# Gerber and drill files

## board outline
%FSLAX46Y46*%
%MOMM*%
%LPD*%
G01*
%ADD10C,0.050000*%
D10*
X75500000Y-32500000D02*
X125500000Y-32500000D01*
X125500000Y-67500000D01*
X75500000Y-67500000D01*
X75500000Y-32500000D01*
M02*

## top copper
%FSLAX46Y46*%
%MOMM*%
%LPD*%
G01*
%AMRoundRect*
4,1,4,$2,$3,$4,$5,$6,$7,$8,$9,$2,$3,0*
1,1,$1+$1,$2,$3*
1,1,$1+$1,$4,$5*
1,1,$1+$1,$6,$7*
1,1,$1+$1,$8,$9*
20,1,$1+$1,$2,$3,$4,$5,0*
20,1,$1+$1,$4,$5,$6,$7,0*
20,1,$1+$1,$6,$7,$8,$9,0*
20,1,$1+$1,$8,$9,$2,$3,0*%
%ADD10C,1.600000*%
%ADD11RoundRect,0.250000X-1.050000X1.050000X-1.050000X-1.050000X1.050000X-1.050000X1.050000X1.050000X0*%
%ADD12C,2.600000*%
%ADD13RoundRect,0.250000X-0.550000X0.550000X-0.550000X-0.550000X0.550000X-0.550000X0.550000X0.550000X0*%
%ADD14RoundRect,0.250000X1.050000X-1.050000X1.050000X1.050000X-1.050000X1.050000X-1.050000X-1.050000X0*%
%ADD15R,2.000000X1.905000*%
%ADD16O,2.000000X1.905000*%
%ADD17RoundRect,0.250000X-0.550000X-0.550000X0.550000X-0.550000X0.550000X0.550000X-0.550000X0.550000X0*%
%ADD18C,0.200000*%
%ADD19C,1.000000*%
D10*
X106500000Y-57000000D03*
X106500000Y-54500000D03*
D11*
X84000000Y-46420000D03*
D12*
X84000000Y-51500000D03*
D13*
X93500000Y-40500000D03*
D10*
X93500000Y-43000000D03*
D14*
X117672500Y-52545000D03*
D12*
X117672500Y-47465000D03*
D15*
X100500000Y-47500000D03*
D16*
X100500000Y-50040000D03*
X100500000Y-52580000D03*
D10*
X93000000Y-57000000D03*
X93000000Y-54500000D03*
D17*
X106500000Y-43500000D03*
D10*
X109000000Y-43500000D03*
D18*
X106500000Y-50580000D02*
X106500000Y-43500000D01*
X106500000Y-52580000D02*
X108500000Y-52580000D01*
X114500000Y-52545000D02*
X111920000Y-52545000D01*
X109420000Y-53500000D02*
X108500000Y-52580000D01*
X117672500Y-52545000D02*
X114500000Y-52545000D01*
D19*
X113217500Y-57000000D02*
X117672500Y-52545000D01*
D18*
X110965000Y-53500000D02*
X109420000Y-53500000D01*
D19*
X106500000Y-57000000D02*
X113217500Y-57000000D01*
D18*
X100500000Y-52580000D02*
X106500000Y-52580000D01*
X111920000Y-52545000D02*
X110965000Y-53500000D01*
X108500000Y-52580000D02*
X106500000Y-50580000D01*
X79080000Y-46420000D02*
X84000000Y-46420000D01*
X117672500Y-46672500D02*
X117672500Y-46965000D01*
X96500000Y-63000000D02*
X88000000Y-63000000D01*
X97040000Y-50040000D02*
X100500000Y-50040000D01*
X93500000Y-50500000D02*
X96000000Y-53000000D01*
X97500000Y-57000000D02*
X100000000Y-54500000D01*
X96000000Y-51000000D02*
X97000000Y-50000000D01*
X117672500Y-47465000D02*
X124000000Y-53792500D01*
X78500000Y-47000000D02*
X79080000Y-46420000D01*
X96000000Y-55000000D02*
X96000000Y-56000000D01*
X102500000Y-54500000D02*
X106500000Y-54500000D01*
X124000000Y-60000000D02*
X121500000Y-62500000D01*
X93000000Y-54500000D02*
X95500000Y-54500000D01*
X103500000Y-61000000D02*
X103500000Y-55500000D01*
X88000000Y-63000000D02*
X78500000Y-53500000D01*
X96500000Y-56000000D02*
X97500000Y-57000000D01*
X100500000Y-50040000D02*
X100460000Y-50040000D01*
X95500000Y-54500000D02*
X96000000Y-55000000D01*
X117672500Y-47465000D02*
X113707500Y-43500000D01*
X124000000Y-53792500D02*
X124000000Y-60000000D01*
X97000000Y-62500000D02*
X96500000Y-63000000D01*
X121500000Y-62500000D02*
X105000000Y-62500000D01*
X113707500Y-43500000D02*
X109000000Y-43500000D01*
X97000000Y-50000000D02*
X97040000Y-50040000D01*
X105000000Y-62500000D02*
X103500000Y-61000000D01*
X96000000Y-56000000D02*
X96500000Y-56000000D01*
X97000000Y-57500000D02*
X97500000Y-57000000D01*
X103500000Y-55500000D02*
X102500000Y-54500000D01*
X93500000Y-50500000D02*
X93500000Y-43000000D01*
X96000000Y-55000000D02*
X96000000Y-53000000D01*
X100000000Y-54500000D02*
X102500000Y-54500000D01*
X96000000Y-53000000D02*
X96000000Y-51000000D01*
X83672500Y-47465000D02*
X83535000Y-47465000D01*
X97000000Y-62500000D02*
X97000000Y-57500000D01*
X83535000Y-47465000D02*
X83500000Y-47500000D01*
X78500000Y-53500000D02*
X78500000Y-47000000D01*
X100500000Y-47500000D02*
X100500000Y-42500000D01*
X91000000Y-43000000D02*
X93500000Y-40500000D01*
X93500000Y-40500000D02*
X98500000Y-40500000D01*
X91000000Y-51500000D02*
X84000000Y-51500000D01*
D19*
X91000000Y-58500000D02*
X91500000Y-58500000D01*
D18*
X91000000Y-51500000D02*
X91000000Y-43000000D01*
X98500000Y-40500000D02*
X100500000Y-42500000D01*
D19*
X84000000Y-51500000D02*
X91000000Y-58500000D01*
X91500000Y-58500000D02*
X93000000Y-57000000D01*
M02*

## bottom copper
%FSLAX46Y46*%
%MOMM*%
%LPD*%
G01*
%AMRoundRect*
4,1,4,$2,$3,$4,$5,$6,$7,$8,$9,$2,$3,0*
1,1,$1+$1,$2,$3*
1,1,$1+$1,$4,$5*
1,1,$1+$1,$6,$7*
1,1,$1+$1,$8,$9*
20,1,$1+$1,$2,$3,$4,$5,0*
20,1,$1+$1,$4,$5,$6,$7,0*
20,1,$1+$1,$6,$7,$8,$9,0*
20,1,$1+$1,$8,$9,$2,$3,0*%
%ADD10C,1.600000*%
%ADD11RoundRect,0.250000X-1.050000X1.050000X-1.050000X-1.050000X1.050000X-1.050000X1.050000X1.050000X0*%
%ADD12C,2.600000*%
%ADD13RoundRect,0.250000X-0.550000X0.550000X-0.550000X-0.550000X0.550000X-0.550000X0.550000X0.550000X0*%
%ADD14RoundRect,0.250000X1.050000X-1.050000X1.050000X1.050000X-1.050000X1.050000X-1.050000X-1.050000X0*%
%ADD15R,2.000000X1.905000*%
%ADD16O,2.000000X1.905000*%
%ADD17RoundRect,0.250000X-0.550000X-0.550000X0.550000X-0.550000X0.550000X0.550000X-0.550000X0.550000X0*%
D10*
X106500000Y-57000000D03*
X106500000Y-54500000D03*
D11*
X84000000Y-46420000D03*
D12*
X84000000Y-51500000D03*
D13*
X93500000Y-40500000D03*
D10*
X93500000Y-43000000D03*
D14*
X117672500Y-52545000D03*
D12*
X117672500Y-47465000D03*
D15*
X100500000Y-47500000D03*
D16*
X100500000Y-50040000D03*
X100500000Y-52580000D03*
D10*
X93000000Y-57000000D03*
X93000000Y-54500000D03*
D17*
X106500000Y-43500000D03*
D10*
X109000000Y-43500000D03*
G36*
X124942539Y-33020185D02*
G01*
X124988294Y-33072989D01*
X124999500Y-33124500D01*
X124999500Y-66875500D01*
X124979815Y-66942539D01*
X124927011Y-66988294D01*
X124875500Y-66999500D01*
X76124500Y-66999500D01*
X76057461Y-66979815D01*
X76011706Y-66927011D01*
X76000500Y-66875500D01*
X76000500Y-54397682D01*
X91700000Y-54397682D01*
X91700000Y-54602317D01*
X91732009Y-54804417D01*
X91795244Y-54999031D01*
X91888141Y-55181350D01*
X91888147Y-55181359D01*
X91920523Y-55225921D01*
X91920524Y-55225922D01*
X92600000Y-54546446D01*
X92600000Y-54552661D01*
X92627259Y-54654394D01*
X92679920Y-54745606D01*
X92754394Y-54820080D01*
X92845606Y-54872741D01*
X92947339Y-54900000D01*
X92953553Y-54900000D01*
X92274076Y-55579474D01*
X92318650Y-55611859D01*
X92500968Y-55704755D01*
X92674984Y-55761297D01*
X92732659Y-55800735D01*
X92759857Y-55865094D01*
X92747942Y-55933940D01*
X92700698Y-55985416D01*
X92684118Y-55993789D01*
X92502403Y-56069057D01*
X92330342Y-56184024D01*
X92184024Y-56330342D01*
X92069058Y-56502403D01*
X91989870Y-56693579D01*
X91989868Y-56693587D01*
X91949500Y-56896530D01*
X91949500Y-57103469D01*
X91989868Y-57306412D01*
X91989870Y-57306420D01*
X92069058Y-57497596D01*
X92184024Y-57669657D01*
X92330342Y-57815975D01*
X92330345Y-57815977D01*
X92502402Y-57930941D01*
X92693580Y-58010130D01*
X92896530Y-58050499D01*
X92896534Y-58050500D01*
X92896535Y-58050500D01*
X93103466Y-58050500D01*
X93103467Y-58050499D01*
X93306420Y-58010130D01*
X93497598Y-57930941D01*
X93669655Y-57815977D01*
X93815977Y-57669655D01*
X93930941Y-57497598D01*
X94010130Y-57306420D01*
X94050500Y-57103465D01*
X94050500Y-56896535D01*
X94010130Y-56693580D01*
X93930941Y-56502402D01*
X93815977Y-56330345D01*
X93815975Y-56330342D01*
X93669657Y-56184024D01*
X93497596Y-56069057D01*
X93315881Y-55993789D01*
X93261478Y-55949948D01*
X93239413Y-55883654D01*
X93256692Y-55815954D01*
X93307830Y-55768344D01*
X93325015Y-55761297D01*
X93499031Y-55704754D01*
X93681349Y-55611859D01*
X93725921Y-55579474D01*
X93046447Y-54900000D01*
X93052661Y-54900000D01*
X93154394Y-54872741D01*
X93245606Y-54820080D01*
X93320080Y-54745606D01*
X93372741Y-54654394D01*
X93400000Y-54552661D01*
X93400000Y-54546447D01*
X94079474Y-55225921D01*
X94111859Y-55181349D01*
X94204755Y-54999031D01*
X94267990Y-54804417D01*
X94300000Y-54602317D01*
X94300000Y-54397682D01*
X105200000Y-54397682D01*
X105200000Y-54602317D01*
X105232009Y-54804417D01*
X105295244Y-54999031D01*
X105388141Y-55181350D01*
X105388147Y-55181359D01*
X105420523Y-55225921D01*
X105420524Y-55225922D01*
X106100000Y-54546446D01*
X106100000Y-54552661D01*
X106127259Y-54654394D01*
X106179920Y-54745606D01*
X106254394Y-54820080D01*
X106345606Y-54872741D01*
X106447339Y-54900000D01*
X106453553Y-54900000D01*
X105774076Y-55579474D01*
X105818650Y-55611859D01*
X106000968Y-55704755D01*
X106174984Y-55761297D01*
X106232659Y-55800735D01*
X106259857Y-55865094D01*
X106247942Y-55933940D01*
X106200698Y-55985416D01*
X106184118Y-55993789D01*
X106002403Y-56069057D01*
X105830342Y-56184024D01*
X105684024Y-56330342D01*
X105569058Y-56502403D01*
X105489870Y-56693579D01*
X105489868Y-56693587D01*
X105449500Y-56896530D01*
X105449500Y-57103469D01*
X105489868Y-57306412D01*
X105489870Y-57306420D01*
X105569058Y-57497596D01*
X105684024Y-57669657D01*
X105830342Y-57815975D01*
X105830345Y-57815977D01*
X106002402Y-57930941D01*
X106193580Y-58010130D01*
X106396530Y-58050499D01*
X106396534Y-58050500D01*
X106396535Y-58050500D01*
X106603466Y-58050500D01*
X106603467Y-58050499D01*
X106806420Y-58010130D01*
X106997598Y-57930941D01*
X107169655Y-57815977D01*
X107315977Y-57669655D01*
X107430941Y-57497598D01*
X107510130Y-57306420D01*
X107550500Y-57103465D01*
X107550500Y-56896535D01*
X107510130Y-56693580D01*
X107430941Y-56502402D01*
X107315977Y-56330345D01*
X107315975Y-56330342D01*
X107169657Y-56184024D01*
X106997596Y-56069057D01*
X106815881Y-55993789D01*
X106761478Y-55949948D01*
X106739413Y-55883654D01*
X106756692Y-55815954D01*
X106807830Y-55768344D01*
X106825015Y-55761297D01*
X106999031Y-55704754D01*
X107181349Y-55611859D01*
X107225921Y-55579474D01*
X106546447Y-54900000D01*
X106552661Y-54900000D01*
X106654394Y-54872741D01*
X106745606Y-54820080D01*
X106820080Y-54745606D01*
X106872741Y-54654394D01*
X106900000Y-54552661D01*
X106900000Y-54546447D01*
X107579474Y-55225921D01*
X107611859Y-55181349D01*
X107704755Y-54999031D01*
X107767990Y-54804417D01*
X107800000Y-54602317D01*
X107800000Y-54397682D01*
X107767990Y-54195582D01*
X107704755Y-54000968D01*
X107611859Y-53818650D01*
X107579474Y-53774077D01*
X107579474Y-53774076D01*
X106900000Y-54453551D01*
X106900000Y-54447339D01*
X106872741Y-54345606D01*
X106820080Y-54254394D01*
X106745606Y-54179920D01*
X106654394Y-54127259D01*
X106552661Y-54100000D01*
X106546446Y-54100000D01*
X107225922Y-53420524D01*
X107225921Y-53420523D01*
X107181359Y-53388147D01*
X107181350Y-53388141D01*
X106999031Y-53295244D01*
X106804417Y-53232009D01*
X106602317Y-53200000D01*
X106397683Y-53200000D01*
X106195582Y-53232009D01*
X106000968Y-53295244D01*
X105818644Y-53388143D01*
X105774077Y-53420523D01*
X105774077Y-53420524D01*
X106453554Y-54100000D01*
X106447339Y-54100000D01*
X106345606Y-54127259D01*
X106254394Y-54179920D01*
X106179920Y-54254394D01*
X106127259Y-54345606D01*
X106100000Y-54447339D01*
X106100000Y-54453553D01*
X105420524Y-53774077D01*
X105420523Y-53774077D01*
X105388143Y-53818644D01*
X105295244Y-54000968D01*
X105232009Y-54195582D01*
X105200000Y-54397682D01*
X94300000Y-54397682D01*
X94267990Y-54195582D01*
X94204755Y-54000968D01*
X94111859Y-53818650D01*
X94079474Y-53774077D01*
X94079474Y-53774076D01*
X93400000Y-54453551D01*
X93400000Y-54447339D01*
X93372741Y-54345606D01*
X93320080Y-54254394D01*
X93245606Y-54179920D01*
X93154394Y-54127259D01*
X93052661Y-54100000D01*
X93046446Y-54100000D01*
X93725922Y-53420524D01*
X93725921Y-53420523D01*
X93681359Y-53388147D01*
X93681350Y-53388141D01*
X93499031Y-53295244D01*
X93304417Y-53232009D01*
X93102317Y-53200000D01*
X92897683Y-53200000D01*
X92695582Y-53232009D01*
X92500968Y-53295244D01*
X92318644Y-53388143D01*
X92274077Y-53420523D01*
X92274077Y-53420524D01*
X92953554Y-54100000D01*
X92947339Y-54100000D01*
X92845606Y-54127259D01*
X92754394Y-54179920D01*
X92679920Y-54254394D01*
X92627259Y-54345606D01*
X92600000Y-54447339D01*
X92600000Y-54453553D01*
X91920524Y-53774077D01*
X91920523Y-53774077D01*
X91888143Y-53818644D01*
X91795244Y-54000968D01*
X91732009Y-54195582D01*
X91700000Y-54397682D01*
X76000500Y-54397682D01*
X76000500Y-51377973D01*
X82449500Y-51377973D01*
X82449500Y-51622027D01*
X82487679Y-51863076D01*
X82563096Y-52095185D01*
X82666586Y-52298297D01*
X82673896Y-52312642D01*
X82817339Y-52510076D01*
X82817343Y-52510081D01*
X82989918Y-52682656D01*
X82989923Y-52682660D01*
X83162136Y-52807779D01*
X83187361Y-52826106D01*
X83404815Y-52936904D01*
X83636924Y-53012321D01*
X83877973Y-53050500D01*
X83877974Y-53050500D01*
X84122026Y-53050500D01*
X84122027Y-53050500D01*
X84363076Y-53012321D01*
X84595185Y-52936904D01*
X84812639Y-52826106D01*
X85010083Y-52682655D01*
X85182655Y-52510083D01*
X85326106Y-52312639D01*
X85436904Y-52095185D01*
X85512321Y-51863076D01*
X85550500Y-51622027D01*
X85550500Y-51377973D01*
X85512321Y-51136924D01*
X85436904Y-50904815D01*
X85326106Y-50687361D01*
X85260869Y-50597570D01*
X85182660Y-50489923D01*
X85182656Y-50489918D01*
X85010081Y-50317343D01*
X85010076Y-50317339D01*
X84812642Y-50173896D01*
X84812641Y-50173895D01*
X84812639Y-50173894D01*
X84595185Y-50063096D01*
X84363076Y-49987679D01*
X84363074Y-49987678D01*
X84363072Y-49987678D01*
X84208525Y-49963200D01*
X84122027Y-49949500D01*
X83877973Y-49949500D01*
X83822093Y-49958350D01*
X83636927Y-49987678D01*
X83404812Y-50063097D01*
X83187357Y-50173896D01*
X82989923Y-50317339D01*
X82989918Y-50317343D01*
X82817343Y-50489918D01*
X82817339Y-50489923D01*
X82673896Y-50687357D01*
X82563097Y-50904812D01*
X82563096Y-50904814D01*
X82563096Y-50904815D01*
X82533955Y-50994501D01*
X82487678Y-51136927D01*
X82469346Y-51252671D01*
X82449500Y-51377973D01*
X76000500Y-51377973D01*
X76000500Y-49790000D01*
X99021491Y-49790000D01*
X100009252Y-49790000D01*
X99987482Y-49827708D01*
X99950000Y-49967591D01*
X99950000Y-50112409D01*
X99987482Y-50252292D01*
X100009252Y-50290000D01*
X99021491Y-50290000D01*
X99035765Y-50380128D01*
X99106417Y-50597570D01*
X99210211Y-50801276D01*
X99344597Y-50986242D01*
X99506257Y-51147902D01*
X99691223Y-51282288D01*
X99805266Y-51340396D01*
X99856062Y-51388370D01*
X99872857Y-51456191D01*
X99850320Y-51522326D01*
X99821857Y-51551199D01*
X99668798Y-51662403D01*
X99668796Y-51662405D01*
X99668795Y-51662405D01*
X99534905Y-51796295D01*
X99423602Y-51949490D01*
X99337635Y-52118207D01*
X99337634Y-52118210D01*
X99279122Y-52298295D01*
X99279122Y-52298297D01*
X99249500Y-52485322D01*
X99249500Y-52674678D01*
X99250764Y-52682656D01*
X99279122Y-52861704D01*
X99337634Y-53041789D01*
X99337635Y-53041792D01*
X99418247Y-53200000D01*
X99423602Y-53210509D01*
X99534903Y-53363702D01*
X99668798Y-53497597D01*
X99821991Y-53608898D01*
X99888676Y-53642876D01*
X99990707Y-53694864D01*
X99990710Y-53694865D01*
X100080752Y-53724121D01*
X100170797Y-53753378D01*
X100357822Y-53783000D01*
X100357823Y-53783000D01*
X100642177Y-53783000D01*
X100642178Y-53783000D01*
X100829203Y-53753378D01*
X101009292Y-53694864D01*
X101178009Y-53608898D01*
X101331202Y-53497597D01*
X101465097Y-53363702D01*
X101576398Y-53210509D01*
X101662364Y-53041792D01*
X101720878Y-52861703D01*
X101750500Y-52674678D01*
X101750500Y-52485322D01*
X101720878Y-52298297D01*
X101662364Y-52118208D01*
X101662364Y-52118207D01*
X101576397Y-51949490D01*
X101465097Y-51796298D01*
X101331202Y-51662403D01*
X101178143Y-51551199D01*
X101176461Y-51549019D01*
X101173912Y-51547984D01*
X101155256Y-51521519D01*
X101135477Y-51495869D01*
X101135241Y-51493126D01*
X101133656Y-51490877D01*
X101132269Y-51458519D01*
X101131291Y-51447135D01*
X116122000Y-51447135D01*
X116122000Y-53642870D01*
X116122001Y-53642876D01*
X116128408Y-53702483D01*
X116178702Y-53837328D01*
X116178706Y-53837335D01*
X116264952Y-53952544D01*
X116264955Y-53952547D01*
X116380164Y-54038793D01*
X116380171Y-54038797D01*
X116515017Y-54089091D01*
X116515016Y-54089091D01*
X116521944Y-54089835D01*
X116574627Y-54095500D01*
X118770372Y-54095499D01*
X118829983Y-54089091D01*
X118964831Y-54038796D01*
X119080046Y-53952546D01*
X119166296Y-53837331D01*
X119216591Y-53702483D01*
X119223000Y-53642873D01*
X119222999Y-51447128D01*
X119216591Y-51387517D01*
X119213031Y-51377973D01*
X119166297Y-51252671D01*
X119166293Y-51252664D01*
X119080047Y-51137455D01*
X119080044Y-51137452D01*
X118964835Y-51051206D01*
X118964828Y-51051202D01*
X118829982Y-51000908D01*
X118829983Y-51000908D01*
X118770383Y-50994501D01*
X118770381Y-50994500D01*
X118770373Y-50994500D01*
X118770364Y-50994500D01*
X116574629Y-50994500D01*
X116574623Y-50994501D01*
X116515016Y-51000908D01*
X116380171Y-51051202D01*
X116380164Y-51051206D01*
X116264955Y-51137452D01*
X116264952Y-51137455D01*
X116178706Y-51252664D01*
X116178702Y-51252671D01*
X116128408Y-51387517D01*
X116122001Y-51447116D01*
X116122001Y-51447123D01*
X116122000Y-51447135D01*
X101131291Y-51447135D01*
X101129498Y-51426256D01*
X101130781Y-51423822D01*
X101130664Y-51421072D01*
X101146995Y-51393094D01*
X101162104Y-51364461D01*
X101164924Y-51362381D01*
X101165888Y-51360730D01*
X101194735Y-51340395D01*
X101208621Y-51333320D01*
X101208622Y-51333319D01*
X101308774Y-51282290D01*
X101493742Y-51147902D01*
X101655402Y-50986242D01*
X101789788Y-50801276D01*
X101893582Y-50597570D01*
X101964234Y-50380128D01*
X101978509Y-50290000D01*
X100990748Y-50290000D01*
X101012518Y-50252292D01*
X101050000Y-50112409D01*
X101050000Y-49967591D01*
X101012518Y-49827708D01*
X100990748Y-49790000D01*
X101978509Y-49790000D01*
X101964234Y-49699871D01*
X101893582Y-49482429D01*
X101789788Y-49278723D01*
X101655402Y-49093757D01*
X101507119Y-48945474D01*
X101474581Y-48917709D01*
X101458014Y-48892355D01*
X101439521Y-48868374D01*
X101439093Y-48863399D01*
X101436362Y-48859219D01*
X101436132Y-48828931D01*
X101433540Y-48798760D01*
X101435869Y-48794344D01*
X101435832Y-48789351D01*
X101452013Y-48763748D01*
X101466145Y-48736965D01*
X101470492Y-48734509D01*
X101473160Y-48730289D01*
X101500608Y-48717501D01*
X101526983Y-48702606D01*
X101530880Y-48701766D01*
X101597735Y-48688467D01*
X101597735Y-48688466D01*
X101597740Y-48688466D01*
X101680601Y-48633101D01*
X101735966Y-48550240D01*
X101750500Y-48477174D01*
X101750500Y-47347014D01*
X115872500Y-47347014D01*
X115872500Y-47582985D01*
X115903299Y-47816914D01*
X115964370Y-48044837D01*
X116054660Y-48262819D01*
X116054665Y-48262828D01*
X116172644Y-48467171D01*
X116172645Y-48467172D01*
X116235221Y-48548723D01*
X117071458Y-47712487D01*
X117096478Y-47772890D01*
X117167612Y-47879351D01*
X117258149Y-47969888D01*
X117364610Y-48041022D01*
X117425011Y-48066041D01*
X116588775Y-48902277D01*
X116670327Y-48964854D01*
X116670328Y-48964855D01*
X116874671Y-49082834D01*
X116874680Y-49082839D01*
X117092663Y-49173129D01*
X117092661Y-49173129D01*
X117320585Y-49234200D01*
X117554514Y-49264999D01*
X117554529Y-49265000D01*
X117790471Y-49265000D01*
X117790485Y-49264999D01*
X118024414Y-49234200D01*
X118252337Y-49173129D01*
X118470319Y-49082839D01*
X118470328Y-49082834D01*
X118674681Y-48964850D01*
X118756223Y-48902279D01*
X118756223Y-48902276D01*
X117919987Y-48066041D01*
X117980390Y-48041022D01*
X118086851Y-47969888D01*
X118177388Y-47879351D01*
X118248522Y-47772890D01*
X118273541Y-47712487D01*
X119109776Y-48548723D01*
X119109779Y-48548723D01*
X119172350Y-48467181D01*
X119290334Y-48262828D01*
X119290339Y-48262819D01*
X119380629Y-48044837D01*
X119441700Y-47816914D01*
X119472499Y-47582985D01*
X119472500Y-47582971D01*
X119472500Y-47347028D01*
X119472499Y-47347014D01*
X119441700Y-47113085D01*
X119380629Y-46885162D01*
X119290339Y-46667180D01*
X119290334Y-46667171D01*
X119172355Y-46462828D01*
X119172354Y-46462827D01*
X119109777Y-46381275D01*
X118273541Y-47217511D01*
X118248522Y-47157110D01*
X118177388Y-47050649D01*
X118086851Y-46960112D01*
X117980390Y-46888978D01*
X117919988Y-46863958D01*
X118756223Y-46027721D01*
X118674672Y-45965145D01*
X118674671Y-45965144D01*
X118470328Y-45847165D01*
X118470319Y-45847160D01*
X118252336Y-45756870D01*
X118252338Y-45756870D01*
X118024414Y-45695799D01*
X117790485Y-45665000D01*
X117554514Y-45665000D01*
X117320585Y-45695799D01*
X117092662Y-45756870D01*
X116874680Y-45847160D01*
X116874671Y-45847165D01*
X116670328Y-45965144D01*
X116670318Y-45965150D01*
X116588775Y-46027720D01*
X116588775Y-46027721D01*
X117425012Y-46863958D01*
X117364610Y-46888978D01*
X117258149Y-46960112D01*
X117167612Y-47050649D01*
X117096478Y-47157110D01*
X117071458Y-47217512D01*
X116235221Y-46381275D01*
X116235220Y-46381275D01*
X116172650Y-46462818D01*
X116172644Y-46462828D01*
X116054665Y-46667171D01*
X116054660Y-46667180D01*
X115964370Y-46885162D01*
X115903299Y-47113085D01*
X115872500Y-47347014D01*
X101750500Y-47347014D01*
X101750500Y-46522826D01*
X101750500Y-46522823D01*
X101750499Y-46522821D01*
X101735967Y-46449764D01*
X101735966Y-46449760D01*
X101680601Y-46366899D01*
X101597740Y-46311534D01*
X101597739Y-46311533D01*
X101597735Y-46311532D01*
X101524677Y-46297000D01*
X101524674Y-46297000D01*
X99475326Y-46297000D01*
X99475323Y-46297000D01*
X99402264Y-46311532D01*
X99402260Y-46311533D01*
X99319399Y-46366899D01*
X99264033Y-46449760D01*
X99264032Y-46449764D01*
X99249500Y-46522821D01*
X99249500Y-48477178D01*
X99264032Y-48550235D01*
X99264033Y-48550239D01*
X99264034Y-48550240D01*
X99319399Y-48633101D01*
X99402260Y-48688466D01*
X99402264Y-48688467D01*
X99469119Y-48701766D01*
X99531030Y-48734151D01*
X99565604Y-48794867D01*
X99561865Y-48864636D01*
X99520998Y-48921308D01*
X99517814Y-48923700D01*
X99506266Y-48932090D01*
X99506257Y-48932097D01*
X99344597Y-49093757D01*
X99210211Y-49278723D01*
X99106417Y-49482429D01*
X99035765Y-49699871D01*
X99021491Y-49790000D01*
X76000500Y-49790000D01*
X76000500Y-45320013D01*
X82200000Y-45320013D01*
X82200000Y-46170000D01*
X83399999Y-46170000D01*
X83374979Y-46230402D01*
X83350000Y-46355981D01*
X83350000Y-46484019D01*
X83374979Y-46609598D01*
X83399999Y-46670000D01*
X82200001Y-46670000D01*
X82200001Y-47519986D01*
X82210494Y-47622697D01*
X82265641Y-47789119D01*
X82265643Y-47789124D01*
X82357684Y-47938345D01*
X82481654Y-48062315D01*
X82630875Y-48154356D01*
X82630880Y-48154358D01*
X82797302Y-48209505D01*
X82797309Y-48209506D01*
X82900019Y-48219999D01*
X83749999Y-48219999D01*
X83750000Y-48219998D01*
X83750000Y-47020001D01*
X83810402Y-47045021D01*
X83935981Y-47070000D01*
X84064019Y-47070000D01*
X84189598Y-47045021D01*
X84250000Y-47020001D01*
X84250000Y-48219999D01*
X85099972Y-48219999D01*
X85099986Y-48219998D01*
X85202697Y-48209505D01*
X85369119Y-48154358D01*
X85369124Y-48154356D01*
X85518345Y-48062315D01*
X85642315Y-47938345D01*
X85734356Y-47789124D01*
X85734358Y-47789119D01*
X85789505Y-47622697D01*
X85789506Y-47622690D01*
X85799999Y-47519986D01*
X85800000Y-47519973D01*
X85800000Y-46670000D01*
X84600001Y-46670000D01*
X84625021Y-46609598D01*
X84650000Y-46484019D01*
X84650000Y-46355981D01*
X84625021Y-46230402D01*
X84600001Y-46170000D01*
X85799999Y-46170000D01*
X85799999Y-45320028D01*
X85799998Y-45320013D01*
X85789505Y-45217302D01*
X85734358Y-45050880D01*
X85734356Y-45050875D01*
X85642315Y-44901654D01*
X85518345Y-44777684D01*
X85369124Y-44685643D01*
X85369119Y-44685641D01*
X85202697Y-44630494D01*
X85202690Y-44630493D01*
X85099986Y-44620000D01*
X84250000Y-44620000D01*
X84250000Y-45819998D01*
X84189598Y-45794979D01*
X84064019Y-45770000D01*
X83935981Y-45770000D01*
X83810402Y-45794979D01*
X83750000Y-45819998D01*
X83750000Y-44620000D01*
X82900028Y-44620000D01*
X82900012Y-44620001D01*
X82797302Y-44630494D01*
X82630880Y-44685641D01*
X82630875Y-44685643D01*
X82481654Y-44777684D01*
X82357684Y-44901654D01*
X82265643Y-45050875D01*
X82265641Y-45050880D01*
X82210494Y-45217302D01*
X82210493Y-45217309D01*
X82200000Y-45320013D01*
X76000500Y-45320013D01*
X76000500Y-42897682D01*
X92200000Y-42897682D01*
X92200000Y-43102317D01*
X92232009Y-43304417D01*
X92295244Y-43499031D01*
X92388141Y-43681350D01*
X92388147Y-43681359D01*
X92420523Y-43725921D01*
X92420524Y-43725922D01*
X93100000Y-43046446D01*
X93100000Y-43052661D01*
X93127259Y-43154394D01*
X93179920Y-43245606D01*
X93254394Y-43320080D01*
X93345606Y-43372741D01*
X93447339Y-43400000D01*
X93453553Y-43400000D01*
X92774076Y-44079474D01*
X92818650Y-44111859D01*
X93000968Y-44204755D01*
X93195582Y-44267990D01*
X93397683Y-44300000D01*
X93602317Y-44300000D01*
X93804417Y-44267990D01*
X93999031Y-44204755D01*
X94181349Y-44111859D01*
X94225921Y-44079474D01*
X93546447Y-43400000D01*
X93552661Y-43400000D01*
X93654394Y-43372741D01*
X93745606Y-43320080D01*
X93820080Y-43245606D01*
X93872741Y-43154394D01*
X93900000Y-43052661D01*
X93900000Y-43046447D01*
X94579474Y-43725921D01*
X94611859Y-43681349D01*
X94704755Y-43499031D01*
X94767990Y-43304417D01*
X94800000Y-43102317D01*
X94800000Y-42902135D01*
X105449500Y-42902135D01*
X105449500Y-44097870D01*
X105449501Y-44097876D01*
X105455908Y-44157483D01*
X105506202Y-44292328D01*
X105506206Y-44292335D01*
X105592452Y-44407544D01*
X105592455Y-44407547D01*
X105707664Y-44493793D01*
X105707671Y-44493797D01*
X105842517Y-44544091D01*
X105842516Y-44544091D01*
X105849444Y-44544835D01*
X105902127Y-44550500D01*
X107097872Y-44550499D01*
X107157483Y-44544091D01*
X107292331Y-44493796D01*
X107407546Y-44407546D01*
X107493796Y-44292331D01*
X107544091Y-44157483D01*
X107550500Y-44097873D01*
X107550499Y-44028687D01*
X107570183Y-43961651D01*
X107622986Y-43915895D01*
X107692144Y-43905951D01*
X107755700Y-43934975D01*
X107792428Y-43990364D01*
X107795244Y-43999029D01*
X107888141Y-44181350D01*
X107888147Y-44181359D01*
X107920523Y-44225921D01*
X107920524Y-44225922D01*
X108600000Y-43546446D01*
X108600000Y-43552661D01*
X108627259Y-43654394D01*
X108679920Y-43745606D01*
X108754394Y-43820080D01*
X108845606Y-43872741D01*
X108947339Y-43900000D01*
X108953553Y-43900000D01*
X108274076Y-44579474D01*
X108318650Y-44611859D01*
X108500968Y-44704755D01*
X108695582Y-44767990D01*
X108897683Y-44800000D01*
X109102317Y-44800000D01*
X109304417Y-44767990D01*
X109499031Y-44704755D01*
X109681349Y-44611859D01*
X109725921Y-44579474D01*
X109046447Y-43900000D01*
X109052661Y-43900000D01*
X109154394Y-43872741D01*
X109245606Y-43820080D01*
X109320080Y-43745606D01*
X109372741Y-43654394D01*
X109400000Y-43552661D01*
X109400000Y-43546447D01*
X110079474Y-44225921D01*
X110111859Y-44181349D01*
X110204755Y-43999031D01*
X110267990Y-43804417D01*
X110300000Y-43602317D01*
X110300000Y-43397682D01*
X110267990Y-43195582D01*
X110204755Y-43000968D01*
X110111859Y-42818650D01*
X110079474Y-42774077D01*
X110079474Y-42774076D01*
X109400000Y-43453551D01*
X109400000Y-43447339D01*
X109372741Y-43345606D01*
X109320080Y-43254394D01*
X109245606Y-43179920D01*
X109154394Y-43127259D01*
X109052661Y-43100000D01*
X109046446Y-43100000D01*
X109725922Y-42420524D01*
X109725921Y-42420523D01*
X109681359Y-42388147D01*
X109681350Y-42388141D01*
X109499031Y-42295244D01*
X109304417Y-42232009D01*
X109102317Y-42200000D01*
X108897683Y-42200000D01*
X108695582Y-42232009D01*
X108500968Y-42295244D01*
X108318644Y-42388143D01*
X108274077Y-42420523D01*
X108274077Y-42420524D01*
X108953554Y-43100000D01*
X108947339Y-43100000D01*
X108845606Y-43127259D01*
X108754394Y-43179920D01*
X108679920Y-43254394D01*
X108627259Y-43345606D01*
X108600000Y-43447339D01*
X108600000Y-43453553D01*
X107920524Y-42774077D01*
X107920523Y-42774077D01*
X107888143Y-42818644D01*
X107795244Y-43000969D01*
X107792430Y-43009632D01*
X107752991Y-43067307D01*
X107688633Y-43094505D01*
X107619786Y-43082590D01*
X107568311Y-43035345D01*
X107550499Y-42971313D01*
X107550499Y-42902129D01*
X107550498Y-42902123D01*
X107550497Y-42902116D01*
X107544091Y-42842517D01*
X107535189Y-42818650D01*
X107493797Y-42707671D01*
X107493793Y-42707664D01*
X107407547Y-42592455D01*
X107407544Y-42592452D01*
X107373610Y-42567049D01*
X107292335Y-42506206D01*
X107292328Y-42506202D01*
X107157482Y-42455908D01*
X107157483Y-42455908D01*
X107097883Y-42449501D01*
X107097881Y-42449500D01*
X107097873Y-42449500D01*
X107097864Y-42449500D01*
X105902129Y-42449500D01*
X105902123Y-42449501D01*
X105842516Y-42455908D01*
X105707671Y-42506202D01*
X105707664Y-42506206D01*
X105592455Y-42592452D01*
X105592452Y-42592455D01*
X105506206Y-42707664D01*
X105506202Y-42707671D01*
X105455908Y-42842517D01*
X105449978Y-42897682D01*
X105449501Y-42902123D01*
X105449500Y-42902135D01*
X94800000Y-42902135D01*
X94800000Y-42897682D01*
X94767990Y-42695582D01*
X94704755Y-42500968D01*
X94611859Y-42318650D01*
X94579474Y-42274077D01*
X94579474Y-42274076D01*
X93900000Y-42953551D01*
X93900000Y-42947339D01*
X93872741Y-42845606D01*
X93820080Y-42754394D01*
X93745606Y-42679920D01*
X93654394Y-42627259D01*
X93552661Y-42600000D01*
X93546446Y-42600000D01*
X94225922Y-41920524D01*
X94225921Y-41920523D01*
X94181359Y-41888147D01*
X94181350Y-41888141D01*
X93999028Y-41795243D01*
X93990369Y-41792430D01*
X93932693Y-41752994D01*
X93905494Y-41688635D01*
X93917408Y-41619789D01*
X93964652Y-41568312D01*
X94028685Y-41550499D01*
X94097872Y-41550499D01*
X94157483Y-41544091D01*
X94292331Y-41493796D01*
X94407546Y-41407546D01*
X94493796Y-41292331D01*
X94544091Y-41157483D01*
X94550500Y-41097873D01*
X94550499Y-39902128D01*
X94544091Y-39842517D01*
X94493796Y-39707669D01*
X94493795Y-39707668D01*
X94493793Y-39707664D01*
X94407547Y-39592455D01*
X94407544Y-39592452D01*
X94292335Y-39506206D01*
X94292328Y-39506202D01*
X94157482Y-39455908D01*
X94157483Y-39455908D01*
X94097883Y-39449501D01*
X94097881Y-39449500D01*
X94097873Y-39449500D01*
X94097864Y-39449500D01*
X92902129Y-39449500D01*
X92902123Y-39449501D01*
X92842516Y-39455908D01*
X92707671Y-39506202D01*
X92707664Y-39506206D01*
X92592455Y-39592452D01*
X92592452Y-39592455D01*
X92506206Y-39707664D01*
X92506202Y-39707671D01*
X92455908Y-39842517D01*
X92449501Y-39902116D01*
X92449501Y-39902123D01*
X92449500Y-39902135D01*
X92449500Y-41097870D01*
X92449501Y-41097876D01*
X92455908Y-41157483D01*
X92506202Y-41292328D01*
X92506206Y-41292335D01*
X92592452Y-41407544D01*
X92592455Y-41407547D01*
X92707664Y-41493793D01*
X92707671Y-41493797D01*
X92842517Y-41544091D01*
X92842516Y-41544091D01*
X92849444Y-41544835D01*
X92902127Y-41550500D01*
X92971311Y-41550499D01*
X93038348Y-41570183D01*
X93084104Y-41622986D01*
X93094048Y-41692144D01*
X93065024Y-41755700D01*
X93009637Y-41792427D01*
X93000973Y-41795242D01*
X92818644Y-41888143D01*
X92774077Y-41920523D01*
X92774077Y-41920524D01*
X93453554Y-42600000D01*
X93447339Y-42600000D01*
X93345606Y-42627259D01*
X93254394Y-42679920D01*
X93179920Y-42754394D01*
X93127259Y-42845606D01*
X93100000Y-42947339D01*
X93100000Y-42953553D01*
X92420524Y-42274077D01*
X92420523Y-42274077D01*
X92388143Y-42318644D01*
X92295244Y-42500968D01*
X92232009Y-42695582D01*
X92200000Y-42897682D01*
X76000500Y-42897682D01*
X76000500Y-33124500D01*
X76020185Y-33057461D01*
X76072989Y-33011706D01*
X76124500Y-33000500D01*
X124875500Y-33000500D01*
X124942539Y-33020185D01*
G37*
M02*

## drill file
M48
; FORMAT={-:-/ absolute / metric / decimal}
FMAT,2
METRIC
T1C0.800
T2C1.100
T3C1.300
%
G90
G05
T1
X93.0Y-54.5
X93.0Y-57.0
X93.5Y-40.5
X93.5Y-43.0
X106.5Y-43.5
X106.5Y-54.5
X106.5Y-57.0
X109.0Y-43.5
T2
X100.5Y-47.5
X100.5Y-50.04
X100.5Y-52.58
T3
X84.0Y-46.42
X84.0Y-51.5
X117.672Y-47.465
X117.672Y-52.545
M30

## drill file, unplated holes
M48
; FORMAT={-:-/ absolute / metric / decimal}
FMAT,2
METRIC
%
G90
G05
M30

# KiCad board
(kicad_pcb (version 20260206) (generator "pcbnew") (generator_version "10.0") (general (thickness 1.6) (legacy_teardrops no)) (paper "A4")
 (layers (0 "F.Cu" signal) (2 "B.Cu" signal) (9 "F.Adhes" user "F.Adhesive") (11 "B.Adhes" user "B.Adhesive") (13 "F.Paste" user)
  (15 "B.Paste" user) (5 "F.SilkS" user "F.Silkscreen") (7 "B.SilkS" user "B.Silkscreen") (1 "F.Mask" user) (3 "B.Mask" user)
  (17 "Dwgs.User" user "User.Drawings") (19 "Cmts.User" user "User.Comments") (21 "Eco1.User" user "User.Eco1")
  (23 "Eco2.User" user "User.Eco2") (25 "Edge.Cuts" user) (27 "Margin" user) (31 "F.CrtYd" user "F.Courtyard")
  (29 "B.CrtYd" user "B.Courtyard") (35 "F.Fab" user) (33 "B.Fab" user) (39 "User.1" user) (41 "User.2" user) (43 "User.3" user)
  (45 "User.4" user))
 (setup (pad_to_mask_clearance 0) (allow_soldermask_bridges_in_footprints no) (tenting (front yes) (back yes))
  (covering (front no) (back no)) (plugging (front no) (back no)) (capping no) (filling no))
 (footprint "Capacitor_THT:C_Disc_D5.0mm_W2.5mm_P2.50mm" (layer "F.Cu") (at 106.5 57 90)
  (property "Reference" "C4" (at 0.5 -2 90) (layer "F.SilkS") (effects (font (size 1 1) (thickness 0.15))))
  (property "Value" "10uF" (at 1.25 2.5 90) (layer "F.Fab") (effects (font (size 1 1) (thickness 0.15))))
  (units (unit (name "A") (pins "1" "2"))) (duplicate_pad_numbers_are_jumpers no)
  (pad "1" thru_hole circle (at 0 0 90) (size 1.6 1.6) (drill 0.8) (layers "*.Cu" "*.Mask") (remove_unused_layers no) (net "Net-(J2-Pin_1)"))
  (pad "2" thru_hole circle (at 2.5 0 90) (size 1.6 1.6) (drill 0.8) (layers "*.Cu" "*.Mask") (remove_unused_layers no) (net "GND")))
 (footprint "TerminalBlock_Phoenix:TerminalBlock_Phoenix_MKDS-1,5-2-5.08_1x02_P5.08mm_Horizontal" (layer "F.Cu") (at 84 46.42 -90)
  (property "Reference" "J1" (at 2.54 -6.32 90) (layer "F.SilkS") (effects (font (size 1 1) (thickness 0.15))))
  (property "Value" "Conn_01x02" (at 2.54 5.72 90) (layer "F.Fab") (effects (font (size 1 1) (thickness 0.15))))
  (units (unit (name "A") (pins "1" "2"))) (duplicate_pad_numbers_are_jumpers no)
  (pad "1" thru_hole roundrect (at 0 0 270) (size 2.6 2.6) (drill 1.3) (layers "*.Cu" "*.Mask") (remove_unused_layers no)
   (roundrect_rratio 0.096154) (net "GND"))
  (pad "2" thru_hole circle (at 5.08 0 270) (size 2.6 2.6) (drill 1.3) (layers "*.Cu" "*.Mask") (remove_unused_layers no) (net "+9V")))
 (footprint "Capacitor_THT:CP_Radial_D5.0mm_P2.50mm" (layer "F.Cu") (at 93.5 40.5 -90)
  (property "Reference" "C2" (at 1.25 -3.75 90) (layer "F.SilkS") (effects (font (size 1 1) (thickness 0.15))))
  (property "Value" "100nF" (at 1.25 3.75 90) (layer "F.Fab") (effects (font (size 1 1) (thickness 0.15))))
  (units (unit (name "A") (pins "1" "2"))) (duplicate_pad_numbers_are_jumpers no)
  (pad "1" thru_hole roundrect (at 0 0 270) (size 1.6 1.6) (drill 0.8) (layers "*.Cu" "*.Mask") (remove_unused_layers no)
   (roundrect_rratio 0.15625) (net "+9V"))
  (pad "2" thru_hole circle (at 2.5 0 270) (size 1.6 1.6) (drill 0.8) (layers "*.Cu" "*.Mask") (remove_unused_layers no) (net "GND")))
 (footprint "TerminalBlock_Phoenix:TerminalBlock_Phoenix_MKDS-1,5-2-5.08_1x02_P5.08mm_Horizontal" (layer "F.Cu") (at 117.6725 52.545 90)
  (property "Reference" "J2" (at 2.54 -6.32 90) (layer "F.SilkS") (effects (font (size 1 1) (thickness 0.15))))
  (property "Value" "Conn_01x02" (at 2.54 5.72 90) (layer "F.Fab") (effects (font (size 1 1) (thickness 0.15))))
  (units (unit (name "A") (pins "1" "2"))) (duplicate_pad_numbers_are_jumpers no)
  (pad "1" thru_hole roundrect (at 0 0 90) (size 2.6 2.6) (drill 1.3) (layers "*.Cu" "*.Mask") (remove_unused_layers no)
   (roundrect_rratio 0.096154) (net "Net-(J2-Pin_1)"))
  (pad "2" thru_hole circle (at 5.08 0 90) (size 2.6 2.6) (drill 1.3) (layers "*.Cu" "*.Mask") (remove_unused_layers no) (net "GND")))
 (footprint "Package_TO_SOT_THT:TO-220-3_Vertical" (layer "F.Cu") (at 100.5 47.5 -90)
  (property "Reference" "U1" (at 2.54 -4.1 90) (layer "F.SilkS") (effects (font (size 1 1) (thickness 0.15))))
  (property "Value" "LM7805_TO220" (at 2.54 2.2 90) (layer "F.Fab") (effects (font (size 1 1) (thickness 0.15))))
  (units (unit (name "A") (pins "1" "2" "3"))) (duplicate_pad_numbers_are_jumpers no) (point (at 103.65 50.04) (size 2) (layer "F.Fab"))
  (pad "1" thru_hole rect (at 0 0 270) (size 1.905 2) (drill 1.1) (layers "*.Cu" "*.Mask") (remove_unused_layers no) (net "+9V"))
  (pad "2" thru_hole oval (at 2.54 0 270) (size 1.905 2) (drill 1.1) (layers "*.Cu" "*.Mask") (remove_unused_layers no) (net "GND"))
  (pad "3" thru_hole oval (at 5.08 0 270) (size 1.905 2) (drill 1.1) (layers "*.Cu" "*.Mask") (remove_unused_layers no)
   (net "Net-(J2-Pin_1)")))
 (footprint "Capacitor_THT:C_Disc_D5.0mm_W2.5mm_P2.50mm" (layer "F.Cu") (at 93 57 90)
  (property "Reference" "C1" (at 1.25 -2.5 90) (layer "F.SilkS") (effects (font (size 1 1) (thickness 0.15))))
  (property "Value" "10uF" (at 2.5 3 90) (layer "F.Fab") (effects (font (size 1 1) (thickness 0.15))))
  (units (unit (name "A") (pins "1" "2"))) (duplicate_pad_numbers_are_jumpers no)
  (pad "1" thru_hole circle (at 0 0 90) (size 1.6 1.6) (drill 0.8) (layers "*.Cu" "*.Mask") (remove_unused_layers no) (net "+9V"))
  (pad "2" thru_hole circle (at 2.5 0 90) (size 1.6 1.6) (drill 0.8) (layers "*.Cu" "*.Mask") (remove_unused_layers no) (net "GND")))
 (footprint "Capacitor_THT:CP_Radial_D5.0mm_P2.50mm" (layer "F.Cu") (at 106.5 43.5)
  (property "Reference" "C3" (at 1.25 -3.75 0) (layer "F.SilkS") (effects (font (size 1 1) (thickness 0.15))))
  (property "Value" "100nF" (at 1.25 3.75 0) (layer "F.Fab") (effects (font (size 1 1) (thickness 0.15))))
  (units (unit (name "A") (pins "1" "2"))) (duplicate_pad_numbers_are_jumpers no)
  (pad "1" thru_hole roundrect (at 0 0) (size 1.6 1.6) (drill 0.8) (layers "*.Cu" "*.Mask") (remove_unused_layers no)
   (roundrect_rratio 0.15625) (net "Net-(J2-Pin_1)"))
  (pad "2" thru_hole circle (at 2.5 0) (size 1.6 1.6) (drill 0.8) (layers "*.Cu" "*.Mask") (remove_unused_layers no) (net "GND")))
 (gr_rect (start 75.5 32.5) (end 125.5 67.5) (stroke (width 0.05) (type default)) (fill no) (layer "Edge.Cuts"))
 (segment (start 106.5 50.58) (end 106.5 43.5) (width 0.2) (layer "F.Cu") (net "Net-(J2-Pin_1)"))
 (segment (start 106.5 52.58) (end 108.5 52.58) (width 0.2) (layer "F.Cu") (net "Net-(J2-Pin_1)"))
 (segment (start 114.5 52.545) (end 111.92 52.545) (width 0.2) (layer "F.Cu") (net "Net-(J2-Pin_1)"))
 (segment (start 109.42 53.5) (end 108.5 52.58) (width 0.2) (layer "F.Cu") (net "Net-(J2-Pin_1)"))
 (segment (start 117.6725 52.545) (end 114.5 52.545) (width 0.2) (layer "F.Cu") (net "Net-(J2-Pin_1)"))
 (segment (start 113.2175 57) (end 117.6725 52.545) (width 1) (layer "F.Cu") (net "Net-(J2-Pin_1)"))
 (segment (start 110.965 53.5) (end 109.42 53.5) (width 0.2) (layer "F.Cu") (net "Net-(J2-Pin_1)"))
 (segment (start 106.5 57) (end 113.2175 57) (width 1) (layer "F.Cu") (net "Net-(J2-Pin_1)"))
 (segment (start 100.5 52.58) (end 106.5 52.58) (width 0.2) (layer "F.Cu") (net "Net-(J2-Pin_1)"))
 (segment (start 111.92 52.545) (end 110.965 53.5) (width 0.2) (layer "F.Cu") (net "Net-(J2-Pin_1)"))
 (segment (start 108.5 52.58) (end 106.5 50.58) (width 0.2) (layer "F.Cu") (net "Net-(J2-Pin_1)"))
 (segment (start 79.08 46.42) (end 84 46.42) (width 0.2) (layer "F.Cu") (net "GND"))
 (segment (start 117.6725 46.6725) (end 117.6725 46.965) (width 0.2) (layer "F.Cu") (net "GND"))
 (segment (start 96.5 63) (end 88 63) (width 0.2) (layer "F.Cu") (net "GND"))
 (segment (start 97.04 50.04) (end 100.5 50.04) (width 0.2) (layer "F.Cu") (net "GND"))
 (segment (start 93.5 50.5) (end 96 53) (width 0.2) (layer "F.Cu") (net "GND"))
 (segment (start 97.5 57) (end 100 54.5) (width 0.2) (layer "F.Cu") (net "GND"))
 (segment (start 96 51) (end 97 50) (width 0.2) (layer "F.Cu") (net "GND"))
 (segment (start 117.6725 47.465) (end 124 53.7925) (width 0.2) (layer "F.Cu") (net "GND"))
 (segment (start 78.5 47) (end 79.08 46.42) (width 0.2) (layer "F.Cu") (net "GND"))
 (segment (start 96 55) (end 96 56) (width 0.2) (layer "F.Cu") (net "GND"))
 (segment (start 102.5 54.5) (end 106.5 54.5) (width 0.2) (layer "F.Cu") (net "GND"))
 (segment (start 124 60) (end 121.5 62.5) (width 0.2) (layer "F.Cu") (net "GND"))
 (segment (start 93 54.5) (end 95.5 54.5) (width 0.2) (layer "F.Cu") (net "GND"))
 (segment (start 103.5 61) (end 103.5 55.5) (width 0.2) (layer "F.Cu") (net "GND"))
 (segment (start 88 63) (end 78.5 53.5) (width 0.2) (layer "F.Cu") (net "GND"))
 (segment (start 96.5 56) (end 97.5 57) (width 0.2) (layer "F.Cu") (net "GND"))
 (segment (start 100.5 50.04) (end 100.46 50.04) (width 0.2) (layer "F.Cu") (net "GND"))
 (segment (start 95.5 54.5) (end 96 55) (width 0.2) (layer "F.Cu") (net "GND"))
 (segment (start 117.6725 47.465) (end 113.7075 43.5) (width 0.2) (layer "F.Cu") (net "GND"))
 (segment (start 124 53.7925) (end 124 60) (width 0.2) (layer "F.Cu") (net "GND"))
 (segment (start 97 62.5) (end 96.5 63) (width 0.2) (layer "F.Cu") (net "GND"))
 (segment (start 121.5 62.5) (end 105 62.5) (width 0.2) (layer "F.Cu") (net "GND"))
 (segment (start 113.7075 43.5) (end 109 43.5) (width 0.2) (layer "F.Cu") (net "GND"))
 (segment (start 97 50) (end 97.04 50.04) (width 0.2) (layer "F.Cu") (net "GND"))
 (segment (start 105 62.5) (end 103.5 61) (width 0.2) (layer "F.Cu") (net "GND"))
 (segment (start 96 56) (end 96.5 56) (width 0.2) (layer "F.Cu") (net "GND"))
 (segment (start 97 57.5) (end 97.5 57) (width 0.2) (layer "F.Cu") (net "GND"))
 (segment (start 103.5 55.5) (end 102.5 54.5) (width 0.2) (layer "F.Cu") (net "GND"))
 (segment (start 93.5 50.5) (end 93.5 43) (width 0.2) (layer "F.Cu") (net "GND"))
 (segment (start 96 55) (end 96 53) (width 0.2) (layer "F.Cu") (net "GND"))
 (segment (start 100 54.5) (end 102.5 54.5) (width 0.2) (layer "F.Cu") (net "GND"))
 (segment (start 96 53) (end 96 51) (width 0.2) (layer "F.Cu") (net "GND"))
 (segment (start 83.6725 47.465) (end 83.535 47.465) (width 0.2) (layer "F.Cu") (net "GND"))
 (segment (start 97 62.5) (end 97 57.5) (width 0.2) (layer "F.Cu") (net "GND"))
 (segment (start 83.535 47.465) (end 83.5 47.5) (width 0.2) (layer "F.Cu") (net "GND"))
 (segment (start 78.5 53.5) (end 78.5 47) (width 0.2) (layer "F.Cu") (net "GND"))
 (segment (start 100.5 47.5) (end 100.5 42.5) (width 0.2) (layer "F.Cu") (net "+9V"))
 (segment (start 91 43) (end 93.5 40.5) (width 0.2) (layer "F.Cu") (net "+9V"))
 (segment (start 93.5 40.5) (end 98.5 40.5) (width 0.2) (layer "F.Cu") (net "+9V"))
 (segment (start 91 51.5) (end 84 51.5) (width 0.2) (layer "F.Cu") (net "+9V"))
 (segment (start 91 58.5) (end 91.5 58.5) (width 1) (layer "F.Cu") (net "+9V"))
 (segment (start 91 51.5) (end 91 43) (width 0.2) (layer "F.Cu") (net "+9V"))
 (segment (start 98.5 40.5) (end 100.5 42.5) (width 0.2) (layer "F.Cu") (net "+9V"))
 (segment (start 84 51.5) (end 91 58.5) (width 1) (layer "F.Cu") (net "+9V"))
 (segment (start 91.5 58.5) (end 93 57) (width 1) (layer "F.Cu") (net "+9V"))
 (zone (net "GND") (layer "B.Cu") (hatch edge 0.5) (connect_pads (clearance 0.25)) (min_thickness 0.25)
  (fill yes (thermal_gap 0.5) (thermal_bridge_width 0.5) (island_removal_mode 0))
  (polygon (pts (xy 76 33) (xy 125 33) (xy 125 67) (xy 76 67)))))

